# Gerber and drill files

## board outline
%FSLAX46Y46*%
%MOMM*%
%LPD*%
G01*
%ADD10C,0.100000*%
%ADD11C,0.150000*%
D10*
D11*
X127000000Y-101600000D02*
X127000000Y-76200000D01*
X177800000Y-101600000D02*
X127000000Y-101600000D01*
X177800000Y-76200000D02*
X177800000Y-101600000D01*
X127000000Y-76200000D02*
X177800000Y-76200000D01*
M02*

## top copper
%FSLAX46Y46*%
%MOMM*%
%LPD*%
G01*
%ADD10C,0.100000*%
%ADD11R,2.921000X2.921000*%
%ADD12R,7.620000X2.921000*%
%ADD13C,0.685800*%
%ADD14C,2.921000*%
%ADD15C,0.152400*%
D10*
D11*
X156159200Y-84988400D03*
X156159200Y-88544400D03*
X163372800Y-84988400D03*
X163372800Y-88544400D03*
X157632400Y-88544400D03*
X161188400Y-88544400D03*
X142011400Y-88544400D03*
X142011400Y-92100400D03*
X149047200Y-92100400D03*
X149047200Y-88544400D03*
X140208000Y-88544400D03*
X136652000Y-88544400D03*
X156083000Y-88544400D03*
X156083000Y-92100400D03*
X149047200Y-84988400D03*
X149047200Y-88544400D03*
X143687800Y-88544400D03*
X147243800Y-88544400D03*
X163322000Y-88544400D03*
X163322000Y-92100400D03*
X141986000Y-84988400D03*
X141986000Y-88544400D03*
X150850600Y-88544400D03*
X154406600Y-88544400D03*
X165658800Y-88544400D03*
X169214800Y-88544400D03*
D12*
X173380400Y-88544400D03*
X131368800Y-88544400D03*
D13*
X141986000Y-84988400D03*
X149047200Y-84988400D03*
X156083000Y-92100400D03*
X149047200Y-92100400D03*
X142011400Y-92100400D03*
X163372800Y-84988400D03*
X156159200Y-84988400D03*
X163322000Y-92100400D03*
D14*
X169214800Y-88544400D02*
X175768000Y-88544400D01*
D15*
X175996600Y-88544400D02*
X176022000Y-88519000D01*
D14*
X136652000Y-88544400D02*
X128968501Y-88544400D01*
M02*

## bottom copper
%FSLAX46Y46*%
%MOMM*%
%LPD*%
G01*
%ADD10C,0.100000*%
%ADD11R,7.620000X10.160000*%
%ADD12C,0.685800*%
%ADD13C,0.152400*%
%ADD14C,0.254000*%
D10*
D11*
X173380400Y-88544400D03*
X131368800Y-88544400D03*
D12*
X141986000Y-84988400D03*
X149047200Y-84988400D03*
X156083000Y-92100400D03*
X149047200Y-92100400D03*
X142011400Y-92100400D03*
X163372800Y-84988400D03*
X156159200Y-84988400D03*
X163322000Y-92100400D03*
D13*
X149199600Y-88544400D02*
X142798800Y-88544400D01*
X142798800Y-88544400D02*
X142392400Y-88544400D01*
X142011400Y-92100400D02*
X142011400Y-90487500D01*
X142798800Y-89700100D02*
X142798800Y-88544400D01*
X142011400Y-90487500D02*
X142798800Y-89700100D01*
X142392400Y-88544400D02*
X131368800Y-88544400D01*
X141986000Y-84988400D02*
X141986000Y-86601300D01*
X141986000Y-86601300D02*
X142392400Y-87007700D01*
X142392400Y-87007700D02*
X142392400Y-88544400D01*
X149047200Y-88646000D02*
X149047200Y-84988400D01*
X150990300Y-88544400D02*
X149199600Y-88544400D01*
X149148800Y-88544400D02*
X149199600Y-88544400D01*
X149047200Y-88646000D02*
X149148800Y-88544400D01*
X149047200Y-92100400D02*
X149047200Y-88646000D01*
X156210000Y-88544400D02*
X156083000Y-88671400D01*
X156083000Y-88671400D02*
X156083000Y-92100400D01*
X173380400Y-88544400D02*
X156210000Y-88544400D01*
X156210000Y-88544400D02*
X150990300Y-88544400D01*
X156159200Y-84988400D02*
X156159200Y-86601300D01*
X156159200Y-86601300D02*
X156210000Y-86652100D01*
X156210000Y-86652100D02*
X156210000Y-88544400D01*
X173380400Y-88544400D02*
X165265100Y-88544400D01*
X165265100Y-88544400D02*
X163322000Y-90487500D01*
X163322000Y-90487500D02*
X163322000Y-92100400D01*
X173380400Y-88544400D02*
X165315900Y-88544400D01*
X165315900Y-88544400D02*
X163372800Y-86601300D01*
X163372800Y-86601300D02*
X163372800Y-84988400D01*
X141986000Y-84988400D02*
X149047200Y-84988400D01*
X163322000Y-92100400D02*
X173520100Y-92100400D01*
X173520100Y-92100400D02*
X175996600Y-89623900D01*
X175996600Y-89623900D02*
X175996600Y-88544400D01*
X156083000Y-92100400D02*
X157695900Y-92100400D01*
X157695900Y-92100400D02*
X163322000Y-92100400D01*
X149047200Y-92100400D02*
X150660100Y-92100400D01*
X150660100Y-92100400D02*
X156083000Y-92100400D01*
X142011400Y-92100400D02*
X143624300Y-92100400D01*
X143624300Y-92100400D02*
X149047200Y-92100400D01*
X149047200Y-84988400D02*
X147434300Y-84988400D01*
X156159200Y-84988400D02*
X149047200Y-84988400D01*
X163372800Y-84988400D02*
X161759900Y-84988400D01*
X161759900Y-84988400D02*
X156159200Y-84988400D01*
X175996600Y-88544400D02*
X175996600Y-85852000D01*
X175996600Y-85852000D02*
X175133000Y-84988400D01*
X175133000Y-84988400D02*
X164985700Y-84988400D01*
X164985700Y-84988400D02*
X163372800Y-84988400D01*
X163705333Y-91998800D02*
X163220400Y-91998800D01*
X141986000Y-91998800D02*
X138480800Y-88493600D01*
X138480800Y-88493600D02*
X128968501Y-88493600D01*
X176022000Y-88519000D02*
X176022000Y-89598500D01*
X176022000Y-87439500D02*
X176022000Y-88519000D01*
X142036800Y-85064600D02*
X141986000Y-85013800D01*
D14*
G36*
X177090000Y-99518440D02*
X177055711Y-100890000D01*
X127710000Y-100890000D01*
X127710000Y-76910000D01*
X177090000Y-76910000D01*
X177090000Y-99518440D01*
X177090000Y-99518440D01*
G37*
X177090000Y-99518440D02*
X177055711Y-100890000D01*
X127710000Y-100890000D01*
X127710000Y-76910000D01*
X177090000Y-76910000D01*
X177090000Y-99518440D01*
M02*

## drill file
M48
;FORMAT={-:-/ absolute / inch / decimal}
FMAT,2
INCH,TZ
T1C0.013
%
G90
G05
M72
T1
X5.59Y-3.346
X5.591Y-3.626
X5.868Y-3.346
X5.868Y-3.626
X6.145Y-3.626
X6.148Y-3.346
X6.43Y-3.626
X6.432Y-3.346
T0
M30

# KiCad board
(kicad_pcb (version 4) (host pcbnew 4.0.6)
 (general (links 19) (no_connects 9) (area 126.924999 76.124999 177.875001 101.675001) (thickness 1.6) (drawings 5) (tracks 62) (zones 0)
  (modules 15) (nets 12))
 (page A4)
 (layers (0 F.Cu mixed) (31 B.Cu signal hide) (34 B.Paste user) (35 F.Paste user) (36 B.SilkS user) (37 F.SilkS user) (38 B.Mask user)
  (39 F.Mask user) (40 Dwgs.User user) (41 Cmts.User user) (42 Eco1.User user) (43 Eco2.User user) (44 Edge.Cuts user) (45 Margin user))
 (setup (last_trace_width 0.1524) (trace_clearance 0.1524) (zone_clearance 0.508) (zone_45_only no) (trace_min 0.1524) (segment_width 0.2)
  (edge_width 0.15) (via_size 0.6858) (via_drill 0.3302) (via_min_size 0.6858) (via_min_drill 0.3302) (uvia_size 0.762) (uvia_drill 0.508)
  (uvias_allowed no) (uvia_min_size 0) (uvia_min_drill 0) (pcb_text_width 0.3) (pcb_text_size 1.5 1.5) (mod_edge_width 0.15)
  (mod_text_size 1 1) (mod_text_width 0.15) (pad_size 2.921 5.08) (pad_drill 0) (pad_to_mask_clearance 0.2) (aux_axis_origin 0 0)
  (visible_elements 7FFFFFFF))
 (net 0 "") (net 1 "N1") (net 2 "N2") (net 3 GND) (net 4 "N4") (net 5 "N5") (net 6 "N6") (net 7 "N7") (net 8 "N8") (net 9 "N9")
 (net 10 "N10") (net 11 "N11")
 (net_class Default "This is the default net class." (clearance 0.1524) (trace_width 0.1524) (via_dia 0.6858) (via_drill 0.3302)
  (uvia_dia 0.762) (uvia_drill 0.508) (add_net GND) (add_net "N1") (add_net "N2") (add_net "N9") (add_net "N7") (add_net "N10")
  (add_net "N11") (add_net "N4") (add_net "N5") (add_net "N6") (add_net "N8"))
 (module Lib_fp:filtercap (layer F.Cu) (at 167.3098 91.5924)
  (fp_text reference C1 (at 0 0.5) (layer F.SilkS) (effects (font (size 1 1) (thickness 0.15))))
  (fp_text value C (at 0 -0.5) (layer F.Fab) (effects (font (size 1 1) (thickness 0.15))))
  (pad 1 smd rect (at -1.651 -3.048) (size 2.921 2.921) (layers F.Cu F.Paste F.Mask) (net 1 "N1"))
  (pad 2 smd rect (at 1.905 -3.048) (size 2.921 2.921) (layers F.Cu F.Paste F.Mask) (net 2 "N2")))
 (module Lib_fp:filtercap (layer F.Cu) (at 153.1112 86.6394 270)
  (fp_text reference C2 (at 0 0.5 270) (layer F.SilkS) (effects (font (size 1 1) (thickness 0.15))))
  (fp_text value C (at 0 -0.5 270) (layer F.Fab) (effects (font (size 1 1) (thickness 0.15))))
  (pad 1 smd rect (at -1.651 -3.048 270) (size 2.921 2.921) (layers F.Cu F.Paste F.Mask) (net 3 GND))
  (pad 2 smd rect (at 1.905 -3.048 270) (size 2.921 2.921) (layers F.Cu F.Paste F.Mask) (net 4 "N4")))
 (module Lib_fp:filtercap (layer F.Cu) (at 160.3248 86.6394 270)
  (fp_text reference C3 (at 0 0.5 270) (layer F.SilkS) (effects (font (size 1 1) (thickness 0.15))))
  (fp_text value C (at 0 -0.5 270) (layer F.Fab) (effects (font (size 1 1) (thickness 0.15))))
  (pad 1 smd rect (at -1.651 -3.048 270) (size 2.921 2.921) (layers F.Cu F.Paste F.Mask) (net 3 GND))
  (pad 2 smd rect (at 1.905 -3.048 270) (size 2.921 2.921) (layers F.Cu F.Paste F.Mask) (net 4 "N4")))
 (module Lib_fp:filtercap (layer F.Cu) (at 159.2834 91.5924)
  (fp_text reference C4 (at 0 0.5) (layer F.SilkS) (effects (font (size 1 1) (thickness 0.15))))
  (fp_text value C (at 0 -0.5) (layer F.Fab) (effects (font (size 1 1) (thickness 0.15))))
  (pad 1 smd rect (at -1.651 -3.048) (size 2.921 2.921) (layers F.Cu F.Paste F.Mask) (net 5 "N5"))
  (pad 2 smd rect (at 1.905 -3.048) (size 2.921 2.921) (layers F.Cu F.Paste F.Mask) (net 1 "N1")))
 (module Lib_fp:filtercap (layer F.Cu) (at 138.9634 90.1954 270)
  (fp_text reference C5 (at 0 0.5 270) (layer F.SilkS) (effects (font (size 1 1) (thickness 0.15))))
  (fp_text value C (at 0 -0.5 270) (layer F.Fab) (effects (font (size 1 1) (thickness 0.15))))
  (pad 1 smd rect (at -1.651 -3.048 270) (size 2.921 2.921) (layers F.Cu F.Paste F.Mask) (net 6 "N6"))
  (pad 2 smd rect (at 1.905 -3.048 270) (size 2.921 2.921) (layers F.Cu F.Paste F.Mask) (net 3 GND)))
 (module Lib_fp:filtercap (layer F.Cu) (at 152.0952 90.4494 90)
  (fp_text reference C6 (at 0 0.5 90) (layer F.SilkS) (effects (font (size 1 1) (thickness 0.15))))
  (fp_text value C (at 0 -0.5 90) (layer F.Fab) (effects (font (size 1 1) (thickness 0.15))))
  (pad 1 smd rect (at -1.651 -3.048 90) (size 2.921 2.921) (layers F.Cu F.Paste F.Mask) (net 3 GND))
  (pad 2 smd rect (at 1.905 -3.048 90) (size 2.921 2.921) (layers F.Cu F.Paste F.Mask) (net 6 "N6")))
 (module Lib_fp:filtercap (layer F.Cu) (at 138.557 85.4964 180)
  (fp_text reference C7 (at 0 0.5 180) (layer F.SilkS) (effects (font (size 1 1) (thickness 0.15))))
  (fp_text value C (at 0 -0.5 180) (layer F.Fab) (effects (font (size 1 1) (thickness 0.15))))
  (pad 1 smd rect (at -1.651 -3.048 180) (size 2.921 2.921) (layers F.Cu F.Paste F.Mask) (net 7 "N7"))
  (pad 2 smd rect (at 1.905 -3.048 180) (size 2.921 2.921) (layers F.Cu F.Paste F.Mask) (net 5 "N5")))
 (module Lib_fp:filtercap (layer F.Cu) (at 153.035 90.1954 270)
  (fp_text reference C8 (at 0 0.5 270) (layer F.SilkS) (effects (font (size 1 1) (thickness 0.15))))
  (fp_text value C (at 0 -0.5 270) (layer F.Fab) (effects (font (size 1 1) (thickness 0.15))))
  (pad 1 smd rect (at -1.651 -3.048 270) (size 2.921 2.921) (layers F.Cu F.Paste F.Mask) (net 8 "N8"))
  (pad 2 smd rect (at 1.905 -3.048 270) (size 2.921 2.921) (layers F.Cu F.Paste F.Mask) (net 3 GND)))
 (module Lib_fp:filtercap (layer F.Cu) (at 145.9992 86.6394 270)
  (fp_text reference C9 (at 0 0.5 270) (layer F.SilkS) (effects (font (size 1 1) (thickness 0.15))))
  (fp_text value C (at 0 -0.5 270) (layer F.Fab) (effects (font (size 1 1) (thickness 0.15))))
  (pad 1 smd rect (at -1.651 -3.048 270) (size 2.921 2.921) (layers F.Cu F.Paste F.Mask) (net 3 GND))
  (pad 2 smd rect (at 1.905 -3.048 270) (size 2.921 2.921) (layers F.Cu F.Paste F.Mask) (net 8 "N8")))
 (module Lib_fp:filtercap (layer F.Cu) (at 145.3388 91.5924)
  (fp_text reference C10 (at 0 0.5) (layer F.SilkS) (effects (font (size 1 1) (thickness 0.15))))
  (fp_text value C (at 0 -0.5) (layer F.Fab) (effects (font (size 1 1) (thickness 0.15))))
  (pad 1 smd rect (at -1.651 -3.048) (size 2.921 2.921) (layers F.Cu F.Paste F.Mask) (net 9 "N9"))
  (pad 2 smd rect (at 1.905 -3.048) (size 2.921 2.921) (layers F.Cu F.Paste F.Mask) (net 7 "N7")))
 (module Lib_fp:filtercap (layer F.Cu) (at 160.274 90.1954 270)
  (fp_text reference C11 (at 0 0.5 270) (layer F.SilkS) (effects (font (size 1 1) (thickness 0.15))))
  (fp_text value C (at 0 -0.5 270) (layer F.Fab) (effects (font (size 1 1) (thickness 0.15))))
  (pad 1 smd rect (at -1.651 -3.048 270) (size 2.921 2.921) (layers F.Cu F.Paste F.Mask) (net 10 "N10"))
  (pad 2 smd rect (at 1.905 -3.048 270) (size 2.921 2.921) (layers F.Cu F.Paste F.Mask) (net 3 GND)))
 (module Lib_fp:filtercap (layer F.Cu) (at 138.938 86.6394 270)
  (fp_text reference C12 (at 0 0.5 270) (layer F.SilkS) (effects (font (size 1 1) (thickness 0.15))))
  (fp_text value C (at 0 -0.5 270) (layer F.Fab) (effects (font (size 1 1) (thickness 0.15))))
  (pad 1 smd rect (at -1.651 -3.048 270) (size 2.921 2.921) (layers F.Cu F.Paste F.Mask) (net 3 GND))
  (pad 2 smd rect (at 1.905 -3.048 270) (size 2.921 2.921) (layers F.Cu F.Paste F.Mask) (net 10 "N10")))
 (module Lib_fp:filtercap (layer F.Cu) (at 152.5016 91.5924)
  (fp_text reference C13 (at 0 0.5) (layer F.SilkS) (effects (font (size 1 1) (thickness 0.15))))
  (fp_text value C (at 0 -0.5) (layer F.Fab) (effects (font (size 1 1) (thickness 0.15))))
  (pad 1 smd rect (at -1.651 -3.048) (size 2.921 2.921) (layers F.Cu F.Paste F.Mask) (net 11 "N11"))
  (pad 2 smd rect (at 1.905 -3.048) (size 2.921 2.921) (layers F.Cu F.Paste F.Mask) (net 9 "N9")))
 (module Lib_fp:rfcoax (layer F.Cu) (at 174.6504 90.8304)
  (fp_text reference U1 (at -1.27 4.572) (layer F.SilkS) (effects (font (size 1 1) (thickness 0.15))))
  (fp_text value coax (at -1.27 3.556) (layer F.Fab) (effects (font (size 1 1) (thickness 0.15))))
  (pad 1 smd rect (at -1.27 -2.286) (size 7.62 2.921) (layers F.Cu F.Paste F.Mask) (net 2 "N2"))
  (pad 2 smd rect (at -1.27 -2.286) (size 7.62 10.16) (layers B.Cu B.Paste B.Mask) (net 3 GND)))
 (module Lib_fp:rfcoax (layer F.Cu) (at 132.6388 90.8304)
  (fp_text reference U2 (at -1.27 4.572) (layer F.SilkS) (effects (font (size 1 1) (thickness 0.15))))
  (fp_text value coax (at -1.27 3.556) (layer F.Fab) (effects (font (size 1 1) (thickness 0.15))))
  (pad 1 smd rect (at -1.27 -2.286) (size 7.62 2.921) (layers F.Cu F.Paste F.Mask) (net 11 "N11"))
  (pad 2 smd rect (at -1.27 -2.286) (size 7.62 10.16) (layers B.Cu B.Paste B.Mask) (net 3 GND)))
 (gr_line (start 127 101.6) (end 127 76.2) (layer Edge.Cuts) (width 0.15))
 (gr_line (start 177.8 101.6) (end 127 101.6) (layer Edge.Cuts) (width 0.15))
 (gr_line (start 177.8 76.2) (end 177.8 101.6) (layer Edge.Cuts) (width 0.15))
 (gr_line (start 127 76.2) (end 177.8 76.2) (layer Edge.Cuts) (width 0.15))
 (segment (start 149.1996 88.5444) (end 142.7988 88.5444) (width 0.1524) (layer B.Cu) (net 3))
 (segment (start 142.7988 88.5444) (end 142.3924 88.5444) (width 0.1524) (layer B.Cu) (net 3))
 (segment (start 142.0114 92.1004) (end 142.0114 90.4875) (width 0.1524) (layer B.Cu) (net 3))
 (segment (start 142.7988 89.7001) (end 142.7988 88.5444) (width 0.1524) (layer B.Cu) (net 3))
 (segment (start 142.0114 90.4875) (end 142.7988 89.7001) (width 0.1524) (layer B.Cu) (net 3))
 (segment (start 142.3924 88.5444) (end 131.3688 88.5444) (width 0.1524) (layer B.Cu) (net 3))
 (segment (start 141.986 84.9884) (end 141.986 86.6013) (width 0.1524) (layer B.Cu) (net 3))
 (segment (start 141.986 86.6013) (end 142.3924 87.0077) (width 0.1524) (layer B.Cu) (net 3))
 (segment (start 142.3924 87.0077) (end 142.3924 88.5444) (width 0.1524) (layer B.Cu) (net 3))
 (segment (start 149.0472 88.646) (end 149.0472 84.9884) (width 0.1524) (layer B.Cu) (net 3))
 (segment (start 150.9903 88.5444) (end 149.1996 88.5444) (width 0.1524) (layer B.Cu) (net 3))
 (segment (start 149.1488 88.5444) (end 149.1996 88.5444) (width 0.1524) (layer B.Cu) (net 3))
 (segment (start 149.0472 88.646) (end 149.1488 88.5444) (width 0.1524) (layer B.Cu) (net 3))
 (segment (start 149.0472 92.1004) (end 149.0472 88.646) (width 0.1524) (layer B.Cu) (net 3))
 (segment (start 156.21 88.5444) (end 156.083 88.6714) (width 0.1524) (layer B.Cu) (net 3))
 (segment (start 156.083 88.6714) (end 156.083 92.1004) (width 0.1524) (layer B.Cu) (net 3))
 (segment (start 173.3804 88.5444) (end 156.21 88.5444) (width 0.1524) (layer B.Cu) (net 3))
 (segment (start 156.21 88.5444) (end 150.9903 88.5444) (width 0.1524) (layer B.Cu) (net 3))
 (segment (start 156.1592 84.9884) (end 156.1592 86.6013) (width 0.1524) (layer B.Cu) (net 3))
 (segment (start 156.1592 86.6013) (end 156.21 86.6521) (width 0.1524) (layer B.Cu) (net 3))
 (segment (start 156.21 86.6521) (end 156.21 88.5444) (width 0.1524) (layer B.Cu) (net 3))
 (segment (start 173.3804 88.5444) (end 165.2651 88.5444) (width 0.1524) (layer B.Cu) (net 3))
 (segment (start 165.2651 88.5444) (end 163.322 90.4875) (width 0.1524) (layer B.Cu) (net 3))
 (segment (start 163.322 90.4875) (end 163.322 92.1004) (width 0.1524) (layer B.Cu) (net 3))
 (segment (start 173.3804 88.5444) (end 165.3159 88.5444) (width 0.1524) (layer B.Cu) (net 3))
 (segment (start 165.3159 88.5444) (end 163.3728 86.6013) (width 0.1524) (layer B.Cu) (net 3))
 (segment (start 163.3728 86.6013) (end 163.3728 84.9884) (width 0.1524) (layer B.Cu) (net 3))
 (segment (start 141.986 84.9884) (end 149.0472 84.9884) (width 0.1524) (layer B.Cu) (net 3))
 (via (at 141.986 84.9884) (size 0.6858) (drill 0.3302) (layers F.Cu B.Cu) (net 3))
 (via (at 149.0472 84.9884) (size 0.6858) (drill 0.3302) (layers F.Cu B.Cu) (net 3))
 (segment (start 163.322 92.1004) (end 173.5201 92.1004) (width 0.1524) (layer B.Cu) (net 3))
 (segment (start 173.5201 92.1004) (end 175.9966 89.6239) (width 0.1524) (layer B.Cu) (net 3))
 (segment (start 175.9966 89.6239) (end 175.9966 88.5444) (width 0.1524) (layer B.Cu) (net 3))
 (segment (start 156.083 92.1004) (end 157.6959 92.1004) (width 0.1524) (layer B.Cu) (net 3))
 (segment (start 157.6959 92.1004) (end 163.322 92.1004) (width 0.1524) (layer B.Cu) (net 3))
 (segment (start 149.0472 92.1004) (end 150.6601 92.1004) (width 0.1524) (layer B.Cu) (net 3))
 (segment (start 150.6601 92.1004) (end 156.083 92.1004) (width 0.1524) (layer B.Cu) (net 3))
 (segment (start 142.0114 92.1004) (end 143.6243 92.1004) (width 0.1524) (layer B.Cu) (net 3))
 (segment (start 143.6243 92.1004) (end 149.0472 92.1004) (width 0.1524) (layer B.Cu) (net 3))
 (segment (start 149.0472 84.9884) (end 147.4343 84.9884) (width 0.1524) (layer B.Cu) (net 3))
 (segment (start 156.1592 84.9884) (end 149.0472 84.9884) (width 0.1524) (layer B.Cu) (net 3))
 (segment (start 163.3728 84.9884) (end 161.7599 84.9884) (width 0.1524) (layer B.Cu) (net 3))
 (segment (start 161.7599 84.9884) (end 156.1592 84.9884) (width 0.1524) (layer B.Cu) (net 3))
 (segment (start 175.9966 88.5444) (end 175.9966 85.852) (width 0.1524) (layer B.Cu) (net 3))
 (segment (start 175.9966 85.852) (end 175.133 84.9884) (width 0.1524) (layer B.Cu) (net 3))
 (segment (start 175.133 84.9884) (end 164.9857 84.9884) (width 0.1524) (layer B.Cu) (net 3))
 (segment (start 164.9857 84.9884) (end 163.3728 84.9884) (width 0.1524) (layer B.Cu) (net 3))
 (via (at 156.083 92.1004) (size 0.6858) (drill 0.3302) (layers F.Cu B.Cu) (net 3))
 (via (at 149.0472 92.1004) (size 0.6858) (drill 0.3302) (layers F.Cu B.Cu) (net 3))
 (via (at 142.0114 92.1004) (size 0.6858) (drill 0.3302) (layers F.Cu B.Cu) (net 3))
 (segment (start 163.705333 91.9988) (end 163.2204 91.9988) (width 0.1524) (layer B.Cu) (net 3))
 (via (at 163.3728 84.9884) (size 0.6858) (drill 0.3302) (layers F.Cu B.Cu) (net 3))
 (via (at 156.1592 84.9884) (size 0.6858) (drill 0.3302) (layers F.Cu B.Cu) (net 3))
 (via (at 163.322 92.1004) (size 0.6858) (drill 0.3302) (layers F.Cu B.Cu) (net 3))
 (segment (start 141.986 91.9988) (end 138.4808 88.4936) (width 0.1524) (layer B.Cu) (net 3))
 (segment (start 138.4808 88.4936) (end 128.968501 88.4936) (width 0.1524) (layer B.Cu) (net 3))
 (segment (start 176.022 88.519) (end 176.022 89.5985) (width 0.1524) (layer B.Cu) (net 3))
 (segment (start 176.022 87.4395) (end 176.022 88.519) (width 0.1524) (layer B.Cu) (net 3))
 (segment (start 142.0368 85.0646) (end 141.986 85.0138) (width 0.1524) (layer B.Cu) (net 3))
 (segment (start 169.2148 88.5444) (end 175.768 88.5444) (width 2.921) (layer F.Cu) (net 2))
 (segment (start 175.9966 88.5444) (end 176.022 88.519) (width 0.1524) (layer F.Cu) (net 2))
 (segment (start 136.652 88.5444) (end 128.968501 88.5444) (width 2.921) (layer F.Cu) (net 11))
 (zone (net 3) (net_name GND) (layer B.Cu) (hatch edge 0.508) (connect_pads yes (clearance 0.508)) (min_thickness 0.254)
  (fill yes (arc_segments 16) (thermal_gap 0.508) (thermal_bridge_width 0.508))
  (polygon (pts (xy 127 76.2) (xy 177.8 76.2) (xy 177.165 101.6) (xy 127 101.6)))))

